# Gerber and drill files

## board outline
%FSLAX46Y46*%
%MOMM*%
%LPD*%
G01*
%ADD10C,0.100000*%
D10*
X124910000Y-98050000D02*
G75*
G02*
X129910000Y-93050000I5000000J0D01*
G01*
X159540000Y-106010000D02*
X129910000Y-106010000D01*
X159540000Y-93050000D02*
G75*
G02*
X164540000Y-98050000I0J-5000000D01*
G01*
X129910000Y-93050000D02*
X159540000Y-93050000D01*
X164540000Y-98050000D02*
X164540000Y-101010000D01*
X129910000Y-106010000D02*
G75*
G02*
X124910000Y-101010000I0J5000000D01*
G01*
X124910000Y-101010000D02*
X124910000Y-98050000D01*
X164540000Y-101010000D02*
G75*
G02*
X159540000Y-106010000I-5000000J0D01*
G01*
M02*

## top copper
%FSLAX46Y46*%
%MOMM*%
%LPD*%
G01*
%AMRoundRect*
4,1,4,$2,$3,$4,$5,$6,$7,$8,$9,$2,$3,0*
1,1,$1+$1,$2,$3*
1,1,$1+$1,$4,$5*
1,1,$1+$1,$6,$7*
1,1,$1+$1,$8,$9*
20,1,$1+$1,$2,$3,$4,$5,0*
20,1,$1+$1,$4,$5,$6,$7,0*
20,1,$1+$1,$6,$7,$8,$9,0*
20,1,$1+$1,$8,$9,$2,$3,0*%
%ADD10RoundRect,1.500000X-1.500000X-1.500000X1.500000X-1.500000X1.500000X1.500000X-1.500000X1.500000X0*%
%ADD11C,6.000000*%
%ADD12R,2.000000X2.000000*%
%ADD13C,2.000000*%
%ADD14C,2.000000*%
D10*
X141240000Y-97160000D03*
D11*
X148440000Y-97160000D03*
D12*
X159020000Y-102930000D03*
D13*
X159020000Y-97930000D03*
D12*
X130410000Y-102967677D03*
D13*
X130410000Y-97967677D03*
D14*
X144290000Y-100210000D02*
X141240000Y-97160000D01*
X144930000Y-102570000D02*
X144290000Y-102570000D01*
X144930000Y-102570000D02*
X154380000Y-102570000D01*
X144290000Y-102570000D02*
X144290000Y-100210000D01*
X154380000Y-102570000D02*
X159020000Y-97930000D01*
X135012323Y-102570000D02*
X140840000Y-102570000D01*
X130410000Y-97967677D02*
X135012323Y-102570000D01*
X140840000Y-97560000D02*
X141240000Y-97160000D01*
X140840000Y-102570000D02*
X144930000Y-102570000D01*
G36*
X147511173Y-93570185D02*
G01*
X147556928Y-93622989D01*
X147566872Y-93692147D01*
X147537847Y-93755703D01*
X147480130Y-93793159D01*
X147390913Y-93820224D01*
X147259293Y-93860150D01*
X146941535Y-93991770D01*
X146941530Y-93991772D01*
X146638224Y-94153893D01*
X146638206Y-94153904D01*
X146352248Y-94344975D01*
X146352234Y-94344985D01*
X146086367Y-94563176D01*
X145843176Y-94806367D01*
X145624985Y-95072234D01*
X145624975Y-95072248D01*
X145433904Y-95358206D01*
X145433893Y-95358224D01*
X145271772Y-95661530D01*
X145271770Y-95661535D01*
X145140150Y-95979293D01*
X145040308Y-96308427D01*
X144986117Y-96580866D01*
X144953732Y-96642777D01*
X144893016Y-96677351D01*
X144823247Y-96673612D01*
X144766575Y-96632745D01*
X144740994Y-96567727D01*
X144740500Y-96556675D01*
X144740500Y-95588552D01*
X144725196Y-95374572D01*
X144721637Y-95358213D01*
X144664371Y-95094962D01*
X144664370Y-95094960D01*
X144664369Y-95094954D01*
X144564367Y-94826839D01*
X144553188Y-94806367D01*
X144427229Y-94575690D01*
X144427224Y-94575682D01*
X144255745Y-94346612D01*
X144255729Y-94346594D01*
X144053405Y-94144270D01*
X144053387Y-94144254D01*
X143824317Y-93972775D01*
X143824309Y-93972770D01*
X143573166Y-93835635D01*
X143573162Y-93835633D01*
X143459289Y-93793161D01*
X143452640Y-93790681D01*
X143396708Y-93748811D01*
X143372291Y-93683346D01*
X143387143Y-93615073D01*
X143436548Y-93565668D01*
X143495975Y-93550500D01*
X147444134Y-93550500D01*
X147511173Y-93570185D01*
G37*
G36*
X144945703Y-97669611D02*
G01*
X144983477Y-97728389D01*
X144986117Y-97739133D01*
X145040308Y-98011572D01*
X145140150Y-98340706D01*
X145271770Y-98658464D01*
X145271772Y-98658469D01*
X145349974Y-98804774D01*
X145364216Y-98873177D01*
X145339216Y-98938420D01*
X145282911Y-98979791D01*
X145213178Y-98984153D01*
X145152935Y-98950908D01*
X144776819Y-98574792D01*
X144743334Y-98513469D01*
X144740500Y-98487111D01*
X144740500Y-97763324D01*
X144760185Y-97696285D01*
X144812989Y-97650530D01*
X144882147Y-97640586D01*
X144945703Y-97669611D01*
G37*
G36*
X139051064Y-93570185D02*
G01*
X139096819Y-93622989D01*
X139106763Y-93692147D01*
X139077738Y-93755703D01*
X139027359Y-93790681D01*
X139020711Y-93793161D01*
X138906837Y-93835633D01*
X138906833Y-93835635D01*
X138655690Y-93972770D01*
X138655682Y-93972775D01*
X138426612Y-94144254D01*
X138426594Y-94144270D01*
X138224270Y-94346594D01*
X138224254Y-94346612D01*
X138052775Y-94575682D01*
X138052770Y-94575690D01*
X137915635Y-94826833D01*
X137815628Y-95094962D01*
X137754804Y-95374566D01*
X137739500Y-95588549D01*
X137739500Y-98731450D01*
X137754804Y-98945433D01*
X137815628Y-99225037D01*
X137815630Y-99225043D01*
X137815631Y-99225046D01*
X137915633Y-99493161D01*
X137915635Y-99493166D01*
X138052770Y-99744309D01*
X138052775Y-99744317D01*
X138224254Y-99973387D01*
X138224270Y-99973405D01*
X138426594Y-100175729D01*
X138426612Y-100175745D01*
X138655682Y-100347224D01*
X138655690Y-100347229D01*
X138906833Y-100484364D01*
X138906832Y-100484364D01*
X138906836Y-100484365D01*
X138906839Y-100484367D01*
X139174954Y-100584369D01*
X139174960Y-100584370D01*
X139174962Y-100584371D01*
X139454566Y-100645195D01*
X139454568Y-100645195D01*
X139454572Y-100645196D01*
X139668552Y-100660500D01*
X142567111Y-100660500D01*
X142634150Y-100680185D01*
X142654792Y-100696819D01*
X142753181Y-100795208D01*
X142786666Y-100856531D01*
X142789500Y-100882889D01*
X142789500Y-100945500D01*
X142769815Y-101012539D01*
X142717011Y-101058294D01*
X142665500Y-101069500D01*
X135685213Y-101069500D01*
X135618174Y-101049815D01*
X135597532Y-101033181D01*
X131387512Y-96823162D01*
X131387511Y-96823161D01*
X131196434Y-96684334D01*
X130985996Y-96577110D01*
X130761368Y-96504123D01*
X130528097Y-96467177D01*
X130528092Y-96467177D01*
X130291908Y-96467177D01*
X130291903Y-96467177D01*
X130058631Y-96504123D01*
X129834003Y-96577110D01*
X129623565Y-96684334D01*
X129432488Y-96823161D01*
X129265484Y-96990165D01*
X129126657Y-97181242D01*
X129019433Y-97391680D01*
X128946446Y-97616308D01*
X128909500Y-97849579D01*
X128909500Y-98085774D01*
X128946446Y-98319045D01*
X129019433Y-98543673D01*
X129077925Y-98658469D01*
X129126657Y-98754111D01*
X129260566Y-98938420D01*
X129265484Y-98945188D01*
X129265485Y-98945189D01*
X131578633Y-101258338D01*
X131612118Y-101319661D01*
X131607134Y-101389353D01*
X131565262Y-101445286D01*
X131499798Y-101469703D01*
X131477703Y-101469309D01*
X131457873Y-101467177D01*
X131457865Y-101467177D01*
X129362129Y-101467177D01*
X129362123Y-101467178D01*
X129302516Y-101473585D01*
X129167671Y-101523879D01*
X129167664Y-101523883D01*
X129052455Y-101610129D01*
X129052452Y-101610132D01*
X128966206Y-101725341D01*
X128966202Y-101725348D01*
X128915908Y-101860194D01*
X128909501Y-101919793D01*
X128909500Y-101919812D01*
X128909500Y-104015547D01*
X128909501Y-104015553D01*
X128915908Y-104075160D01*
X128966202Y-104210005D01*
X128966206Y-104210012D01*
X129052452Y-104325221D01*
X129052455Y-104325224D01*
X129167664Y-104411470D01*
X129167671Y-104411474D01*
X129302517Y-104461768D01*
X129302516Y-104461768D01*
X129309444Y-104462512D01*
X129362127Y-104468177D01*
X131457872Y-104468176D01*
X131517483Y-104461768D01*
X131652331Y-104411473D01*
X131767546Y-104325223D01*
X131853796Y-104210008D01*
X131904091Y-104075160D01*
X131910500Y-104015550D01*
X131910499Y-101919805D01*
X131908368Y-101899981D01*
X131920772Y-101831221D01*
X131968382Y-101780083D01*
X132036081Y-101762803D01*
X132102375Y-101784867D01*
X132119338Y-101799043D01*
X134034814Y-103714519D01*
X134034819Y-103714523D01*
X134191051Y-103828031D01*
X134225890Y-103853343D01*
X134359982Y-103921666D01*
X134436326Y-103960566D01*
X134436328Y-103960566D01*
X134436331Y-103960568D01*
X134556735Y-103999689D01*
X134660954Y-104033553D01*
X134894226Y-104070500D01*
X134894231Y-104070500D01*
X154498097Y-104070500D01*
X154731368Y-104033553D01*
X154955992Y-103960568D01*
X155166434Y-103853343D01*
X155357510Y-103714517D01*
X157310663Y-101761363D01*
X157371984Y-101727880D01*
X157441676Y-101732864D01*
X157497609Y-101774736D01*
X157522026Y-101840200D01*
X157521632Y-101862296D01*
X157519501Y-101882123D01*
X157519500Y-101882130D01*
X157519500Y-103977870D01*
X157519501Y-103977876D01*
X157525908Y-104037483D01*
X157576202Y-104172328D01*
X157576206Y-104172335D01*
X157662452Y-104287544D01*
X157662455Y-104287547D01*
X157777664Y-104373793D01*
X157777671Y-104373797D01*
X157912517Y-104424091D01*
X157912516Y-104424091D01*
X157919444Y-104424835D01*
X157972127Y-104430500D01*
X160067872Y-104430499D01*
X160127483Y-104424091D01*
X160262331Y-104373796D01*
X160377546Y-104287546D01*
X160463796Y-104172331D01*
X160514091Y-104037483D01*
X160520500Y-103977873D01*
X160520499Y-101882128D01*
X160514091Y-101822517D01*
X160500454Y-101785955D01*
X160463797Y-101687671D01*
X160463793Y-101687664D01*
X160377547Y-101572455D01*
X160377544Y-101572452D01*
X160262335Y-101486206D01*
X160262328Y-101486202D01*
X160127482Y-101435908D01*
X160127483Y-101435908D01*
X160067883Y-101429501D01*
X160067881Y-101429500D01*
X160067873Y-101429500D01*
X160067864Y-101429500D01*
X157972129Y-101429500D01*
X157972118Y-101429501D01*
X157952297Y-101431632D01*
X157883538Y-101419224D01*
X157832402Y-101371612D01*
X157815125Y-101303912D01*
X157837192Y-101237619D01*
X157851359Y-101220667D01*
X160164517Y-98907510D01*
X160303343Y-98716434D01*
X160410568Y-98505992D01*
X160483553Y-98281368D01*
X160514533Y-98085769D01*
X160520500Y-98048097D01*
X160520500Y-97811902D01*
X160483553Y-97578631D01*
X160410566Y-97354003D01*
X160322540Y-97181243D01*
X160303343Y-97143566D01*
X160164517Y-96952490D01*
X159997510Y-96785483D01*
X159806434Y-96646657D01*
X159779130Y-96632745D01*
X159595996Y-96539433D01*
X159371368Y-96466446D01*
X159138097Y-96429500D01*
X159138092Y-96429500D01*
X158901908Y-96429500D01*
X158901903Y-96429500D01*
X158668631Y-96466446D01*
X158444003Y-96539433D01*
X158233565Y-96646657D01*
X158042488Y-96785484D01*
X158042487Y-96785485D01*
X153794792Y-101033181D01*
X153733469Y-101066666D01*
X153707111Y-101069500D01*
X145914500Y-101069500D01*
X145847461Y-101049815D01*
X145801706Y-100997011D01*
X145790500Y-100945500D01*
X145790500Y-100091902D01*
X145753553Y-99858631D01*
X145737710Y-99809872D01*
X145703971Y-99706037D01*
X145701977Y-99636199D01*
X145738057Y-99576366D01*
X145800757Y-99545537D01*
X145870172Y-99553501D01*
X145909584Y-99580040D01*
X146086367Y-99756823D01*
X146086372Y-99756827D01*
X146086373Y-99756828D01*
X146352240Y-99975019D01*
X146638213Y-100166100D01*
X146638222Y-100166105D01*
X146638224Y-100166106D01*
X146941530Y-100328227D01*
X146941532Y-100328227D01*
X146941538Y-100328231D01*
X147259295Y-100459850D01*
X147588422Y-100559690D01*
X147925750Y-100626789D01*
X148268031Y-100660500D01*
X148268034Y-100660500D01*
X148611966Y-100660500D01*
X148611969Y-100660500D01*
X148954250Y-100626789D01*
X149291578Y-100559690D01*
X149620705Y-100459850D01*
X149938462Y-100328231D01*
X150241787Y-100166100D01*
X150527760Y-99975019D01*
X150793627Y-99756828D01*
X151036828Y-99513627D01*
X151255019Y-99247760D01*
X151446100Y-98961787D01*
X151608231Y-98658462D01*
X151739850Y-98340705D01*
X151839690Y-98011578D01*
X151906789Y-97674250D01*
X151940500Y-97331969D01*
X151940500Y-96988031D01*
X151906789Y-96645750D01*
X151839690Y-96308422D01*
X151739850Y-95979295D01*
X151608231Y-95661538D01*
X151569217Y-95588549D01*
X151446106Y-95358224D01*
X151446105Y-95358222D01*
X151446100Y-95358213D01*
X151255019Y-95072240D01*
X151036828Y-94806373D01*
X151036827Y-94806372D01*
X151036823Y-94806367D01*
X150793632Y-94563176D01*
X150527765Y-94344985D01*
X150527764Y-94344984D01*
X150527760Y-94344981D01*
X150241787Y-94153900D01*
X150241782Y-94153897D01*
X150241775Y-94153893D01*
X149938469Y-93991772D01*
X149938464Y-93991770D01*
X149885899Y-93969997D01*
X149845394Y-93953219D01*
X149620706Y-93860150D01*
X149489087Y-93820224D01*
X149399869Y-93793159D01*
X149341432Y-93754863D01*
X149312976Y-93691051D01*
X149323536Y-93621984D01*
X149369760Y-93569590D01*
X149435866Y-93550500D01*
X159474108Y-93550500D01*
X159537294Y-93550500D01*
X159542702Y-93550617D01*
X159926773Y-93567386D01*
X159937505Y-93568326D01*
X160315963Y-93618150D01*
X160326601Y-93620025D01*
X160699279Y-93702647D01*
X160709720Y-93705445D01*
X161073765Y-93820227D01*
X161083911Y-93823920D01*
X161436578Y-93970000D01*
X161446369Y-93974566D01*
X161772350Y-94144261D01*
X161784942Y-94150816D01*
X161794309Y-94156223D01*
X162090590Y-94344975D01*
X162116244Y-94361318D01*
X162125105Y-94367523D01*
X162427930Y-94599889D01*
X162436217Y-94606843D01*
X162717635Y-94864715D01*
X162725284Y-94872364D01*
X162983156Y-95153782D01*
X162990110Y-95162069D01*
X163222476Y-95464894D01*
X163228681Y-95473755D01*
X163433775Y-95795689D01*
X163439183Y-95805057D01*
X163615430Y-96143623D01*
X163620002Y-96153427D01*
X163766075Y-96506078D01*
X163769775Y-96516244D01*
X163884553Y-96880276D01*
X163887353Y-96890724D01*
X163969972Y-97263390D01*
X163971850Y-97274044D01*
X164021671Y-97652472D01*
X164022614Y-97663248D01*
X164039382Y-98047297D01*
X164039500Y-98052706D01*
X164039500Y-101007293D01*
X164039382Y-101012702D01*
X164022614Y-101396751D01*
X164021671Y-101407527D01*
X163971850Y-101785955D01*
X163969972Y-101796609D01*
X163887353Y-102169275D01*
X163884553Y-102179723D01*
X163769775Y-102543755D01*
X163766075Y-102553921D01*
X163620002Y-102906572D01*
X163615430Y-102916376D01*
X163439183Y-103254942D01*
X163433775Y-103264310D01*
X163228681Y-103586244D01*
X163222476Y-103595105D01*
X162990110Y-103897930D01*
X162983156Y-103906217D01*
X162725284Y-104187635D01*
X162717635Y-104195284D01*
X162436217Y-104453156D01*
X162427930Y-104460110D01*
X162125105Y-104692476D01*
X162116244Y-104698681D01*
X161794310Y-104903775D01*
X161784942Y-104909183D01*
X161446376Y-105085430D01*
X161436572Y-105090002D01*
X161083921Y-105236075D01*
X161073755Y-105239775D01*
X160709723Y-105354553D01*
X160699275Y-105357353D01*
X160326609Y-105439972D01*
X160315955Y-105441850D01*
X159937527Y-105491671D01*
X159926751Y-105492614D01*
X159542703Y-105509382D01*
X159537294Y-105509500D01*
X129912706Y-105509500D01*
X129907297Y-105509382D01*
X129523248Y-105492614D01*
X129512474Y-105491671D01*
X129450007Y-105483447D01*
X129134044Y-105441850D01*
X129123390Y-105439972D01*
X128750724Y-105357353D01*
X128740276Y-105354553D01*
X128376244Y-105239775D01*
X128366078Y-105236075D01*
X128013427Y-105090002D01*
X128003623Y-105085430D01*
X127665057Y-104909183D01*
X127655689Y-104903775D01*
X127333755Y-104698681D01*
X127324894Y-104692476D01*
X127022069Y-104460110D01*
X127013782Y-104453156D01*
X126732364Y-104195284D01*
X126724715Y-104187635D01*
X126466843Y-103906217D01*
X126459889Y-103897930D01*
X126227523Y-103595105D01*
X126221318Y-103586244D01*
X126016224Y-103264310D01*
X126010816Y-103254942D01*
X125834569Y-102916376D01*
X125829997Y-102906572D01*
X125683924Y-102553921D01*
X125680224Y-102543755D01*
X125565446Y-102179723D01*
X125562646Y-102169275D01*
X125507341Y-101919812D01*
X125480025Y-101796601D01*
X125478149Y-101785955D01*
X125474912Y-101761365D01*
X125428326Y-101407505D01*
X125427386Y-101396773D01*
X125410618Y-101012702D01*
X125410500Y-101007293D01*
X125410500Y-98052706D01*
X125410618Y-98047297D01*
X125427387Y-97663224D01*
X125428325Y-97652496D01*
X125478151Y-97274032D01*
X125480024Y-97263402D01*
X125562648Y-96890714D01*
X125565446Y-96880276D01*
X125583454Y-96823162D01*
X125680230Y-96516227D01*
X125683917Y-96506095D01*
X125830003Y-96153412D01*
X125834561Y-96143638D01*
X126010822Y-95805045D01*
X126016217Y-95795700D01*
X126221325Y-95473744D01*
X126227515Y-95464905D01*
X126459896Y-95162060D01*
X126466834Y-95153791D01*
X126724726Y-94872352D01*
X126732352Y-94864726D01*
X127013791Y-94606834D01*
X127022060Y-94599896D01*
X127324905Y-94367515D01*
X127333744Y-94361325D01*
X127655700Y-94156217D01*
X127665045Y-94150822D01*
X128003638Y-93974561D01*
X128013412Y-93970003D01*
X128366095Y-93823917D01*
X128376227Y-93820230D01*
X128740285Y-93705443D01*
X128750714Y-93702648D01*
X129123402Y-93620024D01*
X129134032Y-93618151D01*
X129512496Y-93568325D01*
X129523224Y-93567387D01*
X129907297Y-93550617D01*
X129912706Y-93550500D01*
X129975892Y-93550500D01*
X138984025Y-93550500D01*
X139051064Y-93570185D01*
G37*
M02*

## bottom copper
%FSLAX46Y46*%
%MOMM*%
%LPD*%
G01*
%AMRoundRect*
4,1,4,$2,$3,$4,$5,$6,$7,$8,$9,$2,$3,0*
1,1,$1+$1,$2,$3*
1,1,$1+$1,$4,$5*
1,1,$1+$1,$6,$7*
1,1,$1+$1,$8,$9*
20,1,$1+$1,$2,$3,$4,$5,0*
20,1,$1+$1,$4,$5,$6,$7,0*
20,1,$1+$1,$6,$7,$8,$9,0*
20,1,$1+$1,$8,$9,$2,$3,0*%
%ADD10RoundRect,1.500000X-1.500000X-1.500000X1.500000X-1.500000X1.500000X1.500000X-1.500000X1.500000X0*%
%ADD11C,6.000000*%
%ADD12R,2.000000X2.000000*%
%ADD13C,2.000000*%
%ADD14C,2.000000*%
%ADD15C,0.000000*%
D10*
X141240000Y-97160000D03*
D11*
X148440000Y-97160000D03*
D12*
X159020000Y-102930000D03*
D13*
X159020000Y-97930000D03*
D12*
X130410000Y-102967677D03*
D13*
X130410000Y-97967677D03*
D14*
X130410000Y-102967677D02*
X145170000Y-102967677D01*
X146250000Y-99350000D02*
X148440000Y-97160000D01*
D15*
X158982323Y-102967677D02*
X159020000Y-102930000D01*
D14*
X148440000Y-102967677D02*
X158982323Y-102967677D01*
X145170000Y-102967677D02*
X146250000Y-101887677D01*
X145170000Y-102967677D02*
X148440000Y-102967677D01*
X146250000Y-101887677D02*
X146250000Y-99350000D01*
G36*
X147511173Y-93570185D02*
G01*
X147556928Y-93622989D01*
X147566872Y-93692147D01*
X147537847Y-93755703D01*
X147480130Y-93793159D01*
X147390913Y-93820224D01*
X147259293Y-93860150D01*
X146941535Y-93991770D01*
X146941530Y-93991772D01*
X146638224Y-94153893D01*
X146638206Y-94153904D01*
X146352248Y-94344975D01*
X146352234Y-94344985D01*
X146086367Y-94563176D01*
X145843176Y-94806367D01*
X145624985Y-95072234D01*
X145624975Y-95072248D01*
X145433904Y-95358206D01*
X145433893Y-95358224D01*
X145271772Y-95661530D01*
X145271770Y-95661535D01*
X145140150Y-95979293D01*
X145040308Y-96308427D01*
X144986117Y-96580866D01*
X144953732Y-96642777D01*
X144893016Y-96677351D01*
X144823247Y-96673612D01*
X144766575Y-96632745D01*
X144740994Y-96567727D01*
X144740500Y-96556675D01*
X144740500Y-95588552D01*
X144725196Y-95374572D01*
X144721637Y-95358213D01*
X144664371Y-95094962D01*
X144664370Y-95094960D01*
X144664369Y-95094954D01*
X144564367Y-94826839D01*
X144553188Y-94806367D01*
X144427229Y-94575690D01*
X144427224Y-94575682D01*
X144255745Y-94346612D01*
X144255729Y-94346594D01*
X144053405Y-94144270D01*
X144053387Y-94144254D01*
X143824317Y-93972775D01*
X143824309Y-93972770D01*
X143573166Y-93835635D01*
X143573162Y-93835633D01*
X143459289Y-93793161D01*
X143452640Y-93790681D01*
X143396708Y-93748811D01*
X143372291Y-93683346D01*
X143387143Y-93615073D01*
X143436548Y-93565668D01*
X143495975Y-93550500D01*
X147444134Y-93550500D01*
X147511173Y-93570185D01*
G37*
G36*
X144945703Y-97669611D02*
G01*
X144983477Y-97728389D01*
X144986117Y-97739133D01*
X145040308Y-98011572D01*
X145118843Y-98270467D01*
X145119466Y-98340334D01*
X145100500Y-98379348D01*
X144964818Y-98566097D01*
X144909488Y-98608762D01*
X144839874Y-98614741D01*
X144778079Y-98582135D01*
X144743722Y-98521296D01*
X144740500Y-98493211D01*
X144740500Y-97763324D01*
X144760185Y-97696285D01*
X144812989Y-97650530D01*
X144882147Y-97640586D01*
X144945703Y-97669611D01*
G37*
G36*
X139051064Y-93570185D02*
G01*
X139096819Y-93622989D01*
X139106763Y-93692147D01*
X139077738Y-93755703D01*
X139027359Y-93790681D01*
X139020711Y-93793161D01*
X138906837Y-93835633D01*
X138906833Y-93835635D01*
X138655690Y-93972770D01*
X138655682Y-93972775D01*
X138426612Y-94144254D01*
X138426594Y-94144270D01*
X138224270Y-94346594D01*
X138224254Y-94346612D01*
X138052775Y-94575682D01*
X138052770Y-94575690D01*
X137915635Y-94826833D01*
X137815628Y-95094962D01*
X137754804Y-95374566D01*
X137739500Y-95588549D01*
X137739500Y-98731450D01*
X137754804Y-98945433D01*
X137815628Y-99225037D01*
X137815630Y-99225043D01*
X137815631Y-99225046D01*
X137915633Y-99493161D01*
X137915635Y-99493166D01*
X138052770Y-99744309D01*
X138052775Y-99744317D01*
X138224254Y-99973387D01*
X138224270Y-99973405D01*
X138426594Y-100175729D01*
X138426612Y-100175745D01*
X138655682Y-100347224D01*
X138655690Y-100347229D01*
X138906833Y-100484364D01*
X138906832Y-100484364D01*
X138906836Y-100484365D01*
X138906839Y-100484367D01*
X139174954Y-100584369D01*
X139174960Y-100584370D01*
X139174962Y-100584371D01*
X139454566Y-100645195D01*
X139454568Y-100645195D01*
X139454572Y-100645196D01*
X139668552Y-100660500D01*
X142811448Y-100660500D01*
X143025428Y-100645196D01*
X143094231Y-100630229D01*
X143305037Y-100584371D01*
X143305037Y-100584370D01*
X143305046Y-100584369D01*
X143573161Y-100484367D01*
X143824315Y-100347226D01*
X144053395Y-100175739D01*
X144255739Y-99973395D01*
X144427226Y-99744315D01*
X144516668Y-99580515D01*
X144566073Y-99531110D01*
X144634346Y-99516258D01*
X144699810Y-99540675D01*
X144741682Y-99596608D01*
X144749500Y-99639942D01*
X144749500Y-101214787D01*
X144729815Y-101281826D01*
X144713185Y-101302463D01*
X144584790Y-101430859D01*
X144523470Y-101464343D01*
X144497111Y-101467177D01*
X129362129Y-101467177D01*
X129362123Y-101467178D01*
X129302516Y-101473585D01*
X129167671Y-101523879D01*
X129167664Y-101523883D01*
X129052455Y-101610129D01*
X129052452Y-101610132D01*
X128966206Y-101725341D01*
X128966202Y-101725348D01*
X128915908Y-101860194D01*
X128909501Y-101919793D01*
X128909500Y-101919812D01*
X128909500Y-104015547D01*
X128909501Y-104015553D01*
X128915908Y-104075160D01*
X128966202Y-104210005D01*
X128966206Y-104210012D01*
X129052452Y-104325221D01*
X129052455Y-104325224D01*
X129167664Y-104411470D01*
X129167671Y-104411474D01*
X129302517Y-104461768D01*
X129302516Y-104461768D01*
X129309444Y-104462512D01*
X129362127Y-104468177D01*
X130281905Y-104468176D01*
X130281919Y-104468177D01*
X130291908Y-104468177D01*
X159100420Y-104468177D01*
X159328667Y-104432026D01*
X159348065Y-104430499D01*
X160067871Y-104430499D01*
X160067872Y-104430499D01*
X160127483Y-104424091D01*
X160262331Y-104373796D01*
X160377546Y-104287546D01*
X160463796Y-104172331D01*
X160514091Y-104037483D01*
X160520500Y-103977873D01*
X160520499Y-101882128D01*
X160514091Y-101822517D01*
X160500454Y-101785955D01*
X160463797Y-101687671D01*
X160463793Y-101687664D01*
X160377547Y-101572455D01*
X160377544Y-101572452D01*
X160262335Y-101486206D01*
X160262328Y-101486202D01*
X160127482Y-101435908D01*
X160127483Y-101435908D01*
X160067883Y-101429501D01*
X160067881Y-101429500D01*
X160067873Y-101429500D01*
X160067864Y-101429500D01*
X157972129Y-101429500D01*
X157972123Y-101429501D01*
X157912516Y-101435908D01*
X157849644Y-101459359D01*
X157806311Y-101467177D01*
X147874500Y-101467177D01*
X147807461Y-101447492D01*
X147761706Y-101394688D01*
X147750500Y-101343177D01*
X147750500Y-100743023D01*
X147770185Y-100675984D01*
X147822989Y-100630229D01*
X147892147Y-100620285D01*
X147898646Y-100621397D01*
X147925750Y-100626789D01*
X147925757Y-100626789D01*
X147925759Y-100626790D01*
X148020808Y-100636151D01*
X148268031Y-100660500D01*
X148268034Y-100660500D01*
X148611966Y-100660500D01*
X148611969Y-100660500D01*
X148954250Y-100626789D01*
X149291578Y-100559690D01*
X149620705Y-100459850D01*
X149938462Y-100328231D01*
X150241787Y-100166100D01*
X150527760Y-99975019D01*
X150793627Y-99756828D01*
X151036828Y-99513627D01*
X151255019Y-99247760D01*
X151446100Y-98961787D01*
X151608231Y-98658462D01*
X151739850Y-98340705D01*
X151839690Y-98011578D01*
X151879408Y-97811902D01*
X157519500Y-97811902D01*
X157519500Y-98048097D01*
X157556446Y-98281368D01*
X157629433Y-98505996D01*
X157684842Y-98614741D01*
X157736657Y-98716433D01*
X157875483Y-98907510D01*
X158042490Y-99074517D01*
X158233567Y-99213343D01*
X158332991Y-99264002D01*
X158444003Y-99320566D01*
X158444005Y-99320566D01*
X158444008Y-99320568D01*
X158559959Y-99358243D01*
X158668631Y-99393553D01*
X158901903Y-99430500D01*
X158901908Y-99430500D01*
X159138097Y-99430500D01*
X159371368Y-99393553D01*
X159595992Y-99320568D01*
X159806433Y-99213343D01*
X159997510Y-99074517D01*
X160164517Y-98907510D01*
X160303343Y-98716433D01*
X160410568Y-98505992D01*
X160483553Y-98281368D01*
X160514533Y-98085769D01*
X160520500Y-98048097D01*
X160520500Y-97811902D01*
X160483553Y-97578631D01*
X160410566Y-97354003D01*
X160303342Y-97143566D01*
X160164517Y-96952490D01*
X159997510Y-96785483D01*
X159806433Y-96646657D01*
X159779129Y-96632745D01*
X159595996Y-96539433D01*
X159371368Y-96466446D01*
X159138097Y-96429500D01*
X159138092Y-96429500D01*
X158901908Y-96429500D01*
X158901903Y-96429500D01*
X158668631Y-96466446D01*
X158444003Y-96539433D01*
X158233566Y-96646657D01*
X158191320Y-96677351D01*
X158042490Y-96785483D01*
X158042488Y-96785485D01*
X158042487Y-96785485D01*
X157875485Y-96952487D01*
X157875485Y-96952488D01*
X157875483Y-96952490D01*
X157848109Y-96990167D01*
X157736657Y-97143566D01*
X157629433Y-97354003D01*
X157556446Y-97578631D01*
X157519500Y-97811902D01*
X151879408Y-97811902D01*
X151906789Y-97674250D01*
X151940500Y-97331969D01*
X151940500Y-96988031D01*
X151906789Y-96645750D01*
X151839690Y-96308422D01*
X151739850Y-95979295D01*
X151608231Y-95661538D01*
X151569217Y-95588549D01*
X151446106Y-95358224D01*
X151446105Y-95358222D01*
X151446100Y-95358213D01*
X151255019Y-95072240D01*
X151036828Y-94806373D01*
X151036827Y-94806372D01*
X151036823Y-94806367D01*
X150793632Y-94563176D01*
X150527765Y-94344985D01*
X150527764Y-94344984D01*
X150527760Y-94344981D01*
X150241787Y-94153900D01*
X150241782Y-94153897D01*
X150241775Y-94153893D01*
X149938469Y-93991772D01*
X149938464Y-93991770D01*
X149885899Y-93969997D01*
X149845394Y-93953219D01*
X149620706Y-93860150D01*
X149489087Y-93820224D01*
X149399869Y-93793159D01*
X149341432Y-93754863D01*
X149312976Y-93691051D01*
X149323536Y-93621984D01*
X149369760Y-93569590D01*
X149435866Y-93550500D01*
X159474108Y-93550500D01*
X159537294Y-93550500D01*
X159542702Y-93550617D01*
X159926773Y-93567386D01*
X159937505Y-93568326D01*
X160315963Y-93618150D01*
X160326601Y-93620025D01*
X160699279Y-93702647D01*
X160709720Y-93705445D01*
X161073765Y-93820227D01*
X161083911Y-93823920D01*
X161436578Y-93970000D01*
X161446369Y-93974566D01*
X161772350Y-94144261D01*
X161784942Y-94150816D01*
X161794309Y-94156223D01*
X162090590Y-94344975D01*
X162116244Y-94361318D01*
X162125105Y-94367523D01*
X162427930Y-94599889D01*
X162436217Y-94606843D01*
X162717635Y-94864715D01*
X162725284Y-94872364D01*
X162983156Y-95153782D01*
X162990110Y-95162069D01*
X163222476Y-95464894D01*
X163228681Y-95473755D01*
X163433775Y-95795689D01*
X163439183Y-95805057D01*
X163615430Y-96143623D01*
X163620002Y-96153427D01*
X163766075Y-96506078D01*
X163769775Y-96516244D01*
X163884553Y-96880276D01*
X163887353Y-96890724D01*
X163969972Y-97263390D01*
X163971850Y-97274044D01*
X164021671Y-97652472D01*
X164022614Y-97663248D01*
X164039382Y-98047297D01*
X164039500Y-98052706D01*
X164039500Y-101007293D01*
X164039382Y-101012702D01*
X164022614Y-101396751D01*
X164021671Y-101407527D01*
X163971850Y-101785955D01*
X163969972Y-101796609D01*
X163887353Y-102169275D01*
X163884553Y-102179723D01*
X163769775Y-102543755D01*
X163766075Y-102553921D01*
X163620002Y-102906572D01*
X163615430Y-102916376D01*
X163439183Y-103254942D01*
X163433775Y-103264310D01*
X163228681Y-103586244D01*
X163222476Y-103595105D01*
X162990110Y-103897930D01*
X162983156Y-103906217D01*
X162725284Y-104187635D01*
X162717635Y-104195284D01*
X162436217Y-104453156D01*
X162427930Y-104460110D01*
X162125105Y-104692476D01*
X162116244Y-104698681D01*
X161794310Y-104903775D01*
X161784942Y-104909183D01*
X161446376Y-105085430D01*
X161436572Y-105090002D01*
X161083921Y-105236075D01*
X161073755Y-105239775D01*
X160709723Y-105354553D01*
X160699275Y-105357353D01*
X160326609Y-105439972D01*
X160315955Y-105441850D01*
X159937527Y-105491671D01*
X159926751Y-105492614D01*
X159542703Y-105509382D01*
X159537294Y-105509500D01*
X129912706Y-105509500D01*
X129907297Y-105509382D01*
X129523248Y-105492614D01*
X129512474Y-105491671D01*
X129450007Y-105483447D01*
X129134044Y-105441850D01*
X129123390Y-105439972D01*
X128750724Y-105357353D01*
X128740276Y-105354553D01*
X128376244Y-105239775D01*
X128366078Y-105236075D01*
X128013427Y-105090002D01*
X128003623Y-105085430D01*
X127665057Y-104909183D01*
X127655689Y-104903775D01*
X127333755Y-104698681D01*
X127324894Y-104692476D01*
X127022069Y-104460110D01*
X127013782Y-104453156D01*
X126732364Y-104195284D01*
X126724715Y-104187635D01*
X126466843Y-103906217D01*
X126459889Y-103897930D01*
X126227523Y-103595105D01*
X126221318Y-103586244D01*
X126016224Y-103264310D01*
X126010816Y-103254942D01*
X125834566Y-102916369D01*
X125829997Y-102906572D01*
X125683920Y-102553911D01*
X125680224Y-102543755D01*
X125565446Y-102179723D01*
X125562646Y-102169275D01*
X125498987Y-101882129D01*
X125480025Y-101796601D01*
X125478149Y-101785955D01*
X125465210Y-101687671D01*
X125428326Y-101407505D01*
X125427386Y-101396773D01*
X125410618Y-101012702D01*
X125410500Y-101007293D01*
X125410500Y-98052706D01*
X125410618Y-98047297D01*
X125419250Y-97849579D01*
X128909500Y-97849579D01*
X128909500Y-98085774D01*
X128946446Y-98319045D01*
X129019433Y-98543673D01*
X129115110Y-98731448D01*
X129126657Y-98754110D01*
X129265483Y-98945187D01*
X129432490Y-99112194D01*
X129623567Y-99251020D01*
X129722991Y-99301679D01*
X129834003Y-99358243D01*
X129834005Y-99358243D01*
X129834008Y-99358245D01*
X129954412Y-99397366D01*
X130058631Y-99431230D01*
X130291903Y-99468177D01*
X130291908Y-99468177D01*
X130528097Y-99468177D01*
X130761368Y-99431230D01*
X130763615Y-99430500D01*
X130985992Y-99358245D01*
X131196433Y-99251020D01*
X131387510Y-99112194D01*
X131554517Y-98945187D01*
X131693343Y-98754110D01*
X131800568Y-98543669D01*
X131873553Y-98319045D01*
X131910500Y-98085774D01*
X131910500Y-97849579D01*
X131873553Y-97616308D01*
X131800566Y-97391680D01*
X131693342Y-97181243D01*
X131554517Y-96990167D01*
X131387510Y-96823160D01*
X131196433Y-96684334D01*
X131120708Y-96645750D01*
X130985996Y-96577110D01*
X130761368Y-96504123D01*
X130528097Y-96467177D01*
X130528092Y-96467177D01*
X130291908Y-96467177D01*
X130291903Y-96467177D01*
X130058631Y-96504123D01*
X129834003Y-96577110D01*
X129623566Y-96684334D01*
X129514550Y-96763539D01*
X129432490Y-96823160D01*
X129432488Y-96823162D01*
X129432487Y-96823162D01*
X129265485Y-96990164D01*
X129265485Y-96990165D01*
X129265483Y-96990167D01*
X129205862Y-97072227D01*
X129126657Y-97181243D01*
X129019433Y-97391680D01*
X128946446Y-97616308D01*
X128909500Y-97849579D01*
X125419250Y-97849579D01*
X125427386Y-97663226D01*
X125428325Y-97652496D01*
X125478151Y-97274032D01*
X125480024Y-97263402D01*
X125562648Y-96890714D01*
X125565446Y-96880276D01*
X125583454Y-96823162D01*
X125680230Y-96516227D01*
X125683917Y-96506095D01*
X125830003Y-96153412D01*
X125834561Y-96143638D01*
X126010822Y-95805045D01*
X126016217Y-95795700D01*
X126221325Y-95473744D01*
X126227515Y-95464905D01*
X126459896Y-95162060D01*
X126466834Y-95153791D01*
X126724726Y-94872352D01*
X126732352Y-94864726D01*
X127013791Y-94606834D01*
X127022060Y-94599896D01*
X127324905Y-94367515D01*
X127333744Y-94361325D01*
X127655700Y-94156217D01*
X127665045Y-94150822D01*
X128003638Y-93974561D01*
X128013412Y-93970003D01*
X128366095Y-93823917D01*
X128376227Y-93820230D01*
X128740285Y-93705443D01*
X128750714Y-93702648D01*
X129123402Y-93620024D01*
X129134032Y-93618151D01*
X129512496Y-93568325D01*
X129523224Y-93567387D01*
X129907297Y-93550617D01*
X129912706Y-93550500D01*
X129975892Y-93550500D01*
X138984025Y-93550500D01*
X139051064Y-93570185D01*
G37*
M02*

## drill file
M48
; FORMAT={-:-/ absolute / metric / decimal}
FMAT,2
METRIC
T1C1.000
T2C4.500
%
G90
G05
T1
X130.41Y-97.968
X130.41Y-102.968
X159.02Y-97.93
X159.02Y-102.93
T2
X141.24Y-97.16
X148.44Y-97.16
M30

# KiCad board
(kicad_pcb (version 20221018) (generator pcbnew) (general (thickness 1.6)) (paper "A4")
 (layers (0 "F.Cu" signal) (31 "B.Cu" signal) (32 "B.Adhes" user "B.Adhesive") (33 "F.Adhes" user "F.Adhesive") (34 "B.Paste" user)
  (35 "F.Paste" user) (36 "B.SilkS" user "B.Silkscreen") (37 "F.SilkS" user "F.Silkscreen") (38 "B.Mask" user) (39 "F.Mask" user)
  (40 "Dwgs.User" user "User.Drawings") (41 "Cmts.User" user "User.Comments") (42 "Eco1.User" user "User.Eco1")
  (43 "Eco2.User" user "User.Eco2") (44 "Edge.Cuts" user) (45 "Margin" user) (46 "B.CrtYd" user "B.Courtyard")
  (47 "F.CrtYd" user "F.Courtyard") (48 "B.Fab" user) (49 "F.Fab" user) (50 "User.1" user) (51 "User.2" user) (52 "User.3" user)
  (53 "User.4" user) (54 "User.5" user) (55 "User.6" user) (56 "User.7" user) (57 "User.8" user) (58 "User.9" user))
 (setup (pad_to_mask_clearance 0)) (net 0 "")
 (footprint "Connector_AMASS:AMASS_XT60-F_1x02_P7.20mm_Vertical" (layer "F.Cu") (at 141.24 97.16)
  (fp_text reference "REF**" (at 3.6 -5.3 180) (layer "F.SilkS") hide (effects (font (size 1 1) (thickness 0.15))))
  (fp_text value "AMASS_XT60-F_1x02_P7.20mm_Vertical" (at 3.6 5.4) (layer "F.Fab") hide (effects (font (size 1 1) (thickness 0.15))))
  (pad "1" thru_hole roundrect (at 0 0) (size 6 6) (drill 4.5) (layers "*.Cu" "*.Mask") (roundrect_rratio 0.25))
  (pad "2" thru_hole circle (at 7.2 0) (size 6 6) (drill 4.5) (layers "*.Cu" "*.Mask")))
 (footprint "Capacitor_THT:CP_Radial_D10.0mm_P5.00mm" (layer "F.Cu") (at 159.02 102.93 90)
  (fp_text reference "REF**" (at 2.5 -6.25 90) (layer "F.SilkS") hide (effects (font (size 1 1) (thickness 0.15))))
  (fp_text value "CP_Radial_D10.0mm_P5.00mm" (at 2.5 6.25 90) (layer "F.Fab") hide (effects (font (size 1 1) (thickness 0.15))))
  (pad "1" thru_hole rect (at 0 0 90) (size 2 2) (drill 1) (layers "*.Cu" "*.Mask"))
  (pad "2" thru_hole circle (at 5 0 90) (size 2 2) (drill 1) (layers "*.Cu" "*.Mask")))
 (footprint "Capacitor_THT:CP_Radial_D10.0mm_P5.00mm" (layer "F.Cu") (at 130.41 102.967677 90)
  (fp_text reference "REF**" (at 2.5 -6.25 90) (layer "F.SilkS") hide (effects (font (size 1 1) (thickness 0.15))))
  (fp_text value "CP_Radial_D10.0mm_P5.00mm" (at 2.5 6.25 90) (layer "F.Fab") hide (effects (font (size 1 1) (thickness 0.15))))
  (pad "1" thru_hole rect (at 0 0 90) (size 2 2) (drill 1) (layers "*.Cu" "*.Mask"))
  (pad "2" thru_hole circle (at 5 0 90) (size 2 2) (drill 1) (layers "*.Cu" "*.Mask")))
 (gr_arc (start 124.91 98.05) (mid 126.374466 94.514466) (end 129.91 93.05) (stroke (width 0.1) (type default)) (layer "Edge.Cuts"))
 (gr_line (start 159.54 106.01) (end 129.91 106.01) (stroke (width 0.1) (type default)) (layer "Edge.Cuts"))
 (gr_arc (start 159.54 93.05) (mid 163.075534 94.514466) (end 164.54 98.05) (stroke (width 0.1) (type default)) (layer "Edge.Cuts"))
 (gr_line (start 129.91 93.05) (end 159.54 93.05) (stroke (width 0.1) (type default)) (layer "Edge.Cuts"))
 (gr_line (start 164.54 98.05) (end 164.54 101.01) (stroke (width 0.1) (type default)) (layer "Edge.Cuts"))
 (gr_arc (start 129.91 106.01) (mid 126.374466 104.545534) (end 124.91 101.01) (stroke (width 0.1) (type default)) (layer "Edge.Cuts"))
 (gr_line (start 124.91 101.01) (end 124.91 98.05) (stroke (width 0.1) (type default)) (layer "Edge.Cuts"))
 (gr_arc (start 164.54 101.01) (mid 163.075534 104.545534) (end 159.54 106.01) (stroke (width 0.1) (type default)) (layer "Edge.Cuts"))
 (segment (start 144.29 100.21) (end 141.24 97.16) (width 2) (layer "F.Cu") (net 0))
 (segment (start 144.93 102.57) (end 144.29 102.57) (width 2) (layer "F.Cu") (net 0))
 (segment (start 144.93 102.57) (end 154.38 102.57) (width 2) (layer "F.Cu") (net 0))
 (segment (start 144.29 102.57) (end 144.29 100.21) (width 2) (layer "F.Cu") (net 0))
 (segment (start 154.38 102.57) (end 159.02 97.93) (width 2) (layer "F.Cu") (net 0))
 (segment (start 135.012323 102.57) (end 140.84 102.57) (width 2) (layer "F.Cu") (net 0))
 (segment (start 130.41 97.967677) (end 135.012323 102.57) (width 2) (layer "F.Cu") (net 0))
 (segment (start 140.84 97.56) (end 141.24 97.16) (width 2) (layer "F.Cu") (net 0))
 (segment (start 140.84 102.57) (end 144.93 102.57) (width 2) (layer "F.Cu") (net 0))
 (segment (start 130.41 102.967677) (end 145.17 102.967677) (width 2) (layer "B.Cu") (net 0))
 (segment (start 146.25 99.35) (end 148.44 97.16) (width 2) (layer "B.Cu") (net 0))
 (segment (start 158.982323 102.967677) (end 159.02 102.93) (width 0) (layer "B.Cu") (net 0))
 (segment (start 148.44 102.967677) (end 158.982323 102.967677) (width 2) (layer "B.Cu") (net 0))
 (segment (start 145.17 102.967677) (end 146.25 101.887677) (width 2) (layer "B.Cu") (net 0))
 (segment (start 145.17 102.967677) (end 148.44 102.967677) (width 2) (layer "B.Cu") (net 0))
 (segment (start 146.25 101.887677) (end 146.25 99.35) (width 2) (layer "B.Cu") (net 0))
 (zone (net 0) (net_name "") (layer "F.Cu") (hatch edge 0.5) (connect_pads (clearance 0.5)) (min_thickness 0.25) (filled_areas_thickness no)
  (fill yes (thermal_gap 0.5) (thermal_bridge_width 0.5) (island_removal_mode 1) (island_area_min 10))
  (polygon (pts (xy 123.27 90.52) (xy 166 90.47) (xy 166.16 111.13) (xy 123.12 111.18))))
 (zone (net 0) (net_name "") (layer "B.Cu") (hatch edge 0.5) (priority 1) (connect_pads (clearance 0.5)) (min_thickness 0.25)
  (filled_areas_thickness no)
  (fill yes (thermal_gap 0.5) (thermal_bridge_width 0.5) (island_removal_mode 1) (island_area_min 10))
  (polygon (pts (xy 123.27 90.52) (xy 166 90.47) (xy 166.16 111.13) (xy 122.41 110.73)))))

